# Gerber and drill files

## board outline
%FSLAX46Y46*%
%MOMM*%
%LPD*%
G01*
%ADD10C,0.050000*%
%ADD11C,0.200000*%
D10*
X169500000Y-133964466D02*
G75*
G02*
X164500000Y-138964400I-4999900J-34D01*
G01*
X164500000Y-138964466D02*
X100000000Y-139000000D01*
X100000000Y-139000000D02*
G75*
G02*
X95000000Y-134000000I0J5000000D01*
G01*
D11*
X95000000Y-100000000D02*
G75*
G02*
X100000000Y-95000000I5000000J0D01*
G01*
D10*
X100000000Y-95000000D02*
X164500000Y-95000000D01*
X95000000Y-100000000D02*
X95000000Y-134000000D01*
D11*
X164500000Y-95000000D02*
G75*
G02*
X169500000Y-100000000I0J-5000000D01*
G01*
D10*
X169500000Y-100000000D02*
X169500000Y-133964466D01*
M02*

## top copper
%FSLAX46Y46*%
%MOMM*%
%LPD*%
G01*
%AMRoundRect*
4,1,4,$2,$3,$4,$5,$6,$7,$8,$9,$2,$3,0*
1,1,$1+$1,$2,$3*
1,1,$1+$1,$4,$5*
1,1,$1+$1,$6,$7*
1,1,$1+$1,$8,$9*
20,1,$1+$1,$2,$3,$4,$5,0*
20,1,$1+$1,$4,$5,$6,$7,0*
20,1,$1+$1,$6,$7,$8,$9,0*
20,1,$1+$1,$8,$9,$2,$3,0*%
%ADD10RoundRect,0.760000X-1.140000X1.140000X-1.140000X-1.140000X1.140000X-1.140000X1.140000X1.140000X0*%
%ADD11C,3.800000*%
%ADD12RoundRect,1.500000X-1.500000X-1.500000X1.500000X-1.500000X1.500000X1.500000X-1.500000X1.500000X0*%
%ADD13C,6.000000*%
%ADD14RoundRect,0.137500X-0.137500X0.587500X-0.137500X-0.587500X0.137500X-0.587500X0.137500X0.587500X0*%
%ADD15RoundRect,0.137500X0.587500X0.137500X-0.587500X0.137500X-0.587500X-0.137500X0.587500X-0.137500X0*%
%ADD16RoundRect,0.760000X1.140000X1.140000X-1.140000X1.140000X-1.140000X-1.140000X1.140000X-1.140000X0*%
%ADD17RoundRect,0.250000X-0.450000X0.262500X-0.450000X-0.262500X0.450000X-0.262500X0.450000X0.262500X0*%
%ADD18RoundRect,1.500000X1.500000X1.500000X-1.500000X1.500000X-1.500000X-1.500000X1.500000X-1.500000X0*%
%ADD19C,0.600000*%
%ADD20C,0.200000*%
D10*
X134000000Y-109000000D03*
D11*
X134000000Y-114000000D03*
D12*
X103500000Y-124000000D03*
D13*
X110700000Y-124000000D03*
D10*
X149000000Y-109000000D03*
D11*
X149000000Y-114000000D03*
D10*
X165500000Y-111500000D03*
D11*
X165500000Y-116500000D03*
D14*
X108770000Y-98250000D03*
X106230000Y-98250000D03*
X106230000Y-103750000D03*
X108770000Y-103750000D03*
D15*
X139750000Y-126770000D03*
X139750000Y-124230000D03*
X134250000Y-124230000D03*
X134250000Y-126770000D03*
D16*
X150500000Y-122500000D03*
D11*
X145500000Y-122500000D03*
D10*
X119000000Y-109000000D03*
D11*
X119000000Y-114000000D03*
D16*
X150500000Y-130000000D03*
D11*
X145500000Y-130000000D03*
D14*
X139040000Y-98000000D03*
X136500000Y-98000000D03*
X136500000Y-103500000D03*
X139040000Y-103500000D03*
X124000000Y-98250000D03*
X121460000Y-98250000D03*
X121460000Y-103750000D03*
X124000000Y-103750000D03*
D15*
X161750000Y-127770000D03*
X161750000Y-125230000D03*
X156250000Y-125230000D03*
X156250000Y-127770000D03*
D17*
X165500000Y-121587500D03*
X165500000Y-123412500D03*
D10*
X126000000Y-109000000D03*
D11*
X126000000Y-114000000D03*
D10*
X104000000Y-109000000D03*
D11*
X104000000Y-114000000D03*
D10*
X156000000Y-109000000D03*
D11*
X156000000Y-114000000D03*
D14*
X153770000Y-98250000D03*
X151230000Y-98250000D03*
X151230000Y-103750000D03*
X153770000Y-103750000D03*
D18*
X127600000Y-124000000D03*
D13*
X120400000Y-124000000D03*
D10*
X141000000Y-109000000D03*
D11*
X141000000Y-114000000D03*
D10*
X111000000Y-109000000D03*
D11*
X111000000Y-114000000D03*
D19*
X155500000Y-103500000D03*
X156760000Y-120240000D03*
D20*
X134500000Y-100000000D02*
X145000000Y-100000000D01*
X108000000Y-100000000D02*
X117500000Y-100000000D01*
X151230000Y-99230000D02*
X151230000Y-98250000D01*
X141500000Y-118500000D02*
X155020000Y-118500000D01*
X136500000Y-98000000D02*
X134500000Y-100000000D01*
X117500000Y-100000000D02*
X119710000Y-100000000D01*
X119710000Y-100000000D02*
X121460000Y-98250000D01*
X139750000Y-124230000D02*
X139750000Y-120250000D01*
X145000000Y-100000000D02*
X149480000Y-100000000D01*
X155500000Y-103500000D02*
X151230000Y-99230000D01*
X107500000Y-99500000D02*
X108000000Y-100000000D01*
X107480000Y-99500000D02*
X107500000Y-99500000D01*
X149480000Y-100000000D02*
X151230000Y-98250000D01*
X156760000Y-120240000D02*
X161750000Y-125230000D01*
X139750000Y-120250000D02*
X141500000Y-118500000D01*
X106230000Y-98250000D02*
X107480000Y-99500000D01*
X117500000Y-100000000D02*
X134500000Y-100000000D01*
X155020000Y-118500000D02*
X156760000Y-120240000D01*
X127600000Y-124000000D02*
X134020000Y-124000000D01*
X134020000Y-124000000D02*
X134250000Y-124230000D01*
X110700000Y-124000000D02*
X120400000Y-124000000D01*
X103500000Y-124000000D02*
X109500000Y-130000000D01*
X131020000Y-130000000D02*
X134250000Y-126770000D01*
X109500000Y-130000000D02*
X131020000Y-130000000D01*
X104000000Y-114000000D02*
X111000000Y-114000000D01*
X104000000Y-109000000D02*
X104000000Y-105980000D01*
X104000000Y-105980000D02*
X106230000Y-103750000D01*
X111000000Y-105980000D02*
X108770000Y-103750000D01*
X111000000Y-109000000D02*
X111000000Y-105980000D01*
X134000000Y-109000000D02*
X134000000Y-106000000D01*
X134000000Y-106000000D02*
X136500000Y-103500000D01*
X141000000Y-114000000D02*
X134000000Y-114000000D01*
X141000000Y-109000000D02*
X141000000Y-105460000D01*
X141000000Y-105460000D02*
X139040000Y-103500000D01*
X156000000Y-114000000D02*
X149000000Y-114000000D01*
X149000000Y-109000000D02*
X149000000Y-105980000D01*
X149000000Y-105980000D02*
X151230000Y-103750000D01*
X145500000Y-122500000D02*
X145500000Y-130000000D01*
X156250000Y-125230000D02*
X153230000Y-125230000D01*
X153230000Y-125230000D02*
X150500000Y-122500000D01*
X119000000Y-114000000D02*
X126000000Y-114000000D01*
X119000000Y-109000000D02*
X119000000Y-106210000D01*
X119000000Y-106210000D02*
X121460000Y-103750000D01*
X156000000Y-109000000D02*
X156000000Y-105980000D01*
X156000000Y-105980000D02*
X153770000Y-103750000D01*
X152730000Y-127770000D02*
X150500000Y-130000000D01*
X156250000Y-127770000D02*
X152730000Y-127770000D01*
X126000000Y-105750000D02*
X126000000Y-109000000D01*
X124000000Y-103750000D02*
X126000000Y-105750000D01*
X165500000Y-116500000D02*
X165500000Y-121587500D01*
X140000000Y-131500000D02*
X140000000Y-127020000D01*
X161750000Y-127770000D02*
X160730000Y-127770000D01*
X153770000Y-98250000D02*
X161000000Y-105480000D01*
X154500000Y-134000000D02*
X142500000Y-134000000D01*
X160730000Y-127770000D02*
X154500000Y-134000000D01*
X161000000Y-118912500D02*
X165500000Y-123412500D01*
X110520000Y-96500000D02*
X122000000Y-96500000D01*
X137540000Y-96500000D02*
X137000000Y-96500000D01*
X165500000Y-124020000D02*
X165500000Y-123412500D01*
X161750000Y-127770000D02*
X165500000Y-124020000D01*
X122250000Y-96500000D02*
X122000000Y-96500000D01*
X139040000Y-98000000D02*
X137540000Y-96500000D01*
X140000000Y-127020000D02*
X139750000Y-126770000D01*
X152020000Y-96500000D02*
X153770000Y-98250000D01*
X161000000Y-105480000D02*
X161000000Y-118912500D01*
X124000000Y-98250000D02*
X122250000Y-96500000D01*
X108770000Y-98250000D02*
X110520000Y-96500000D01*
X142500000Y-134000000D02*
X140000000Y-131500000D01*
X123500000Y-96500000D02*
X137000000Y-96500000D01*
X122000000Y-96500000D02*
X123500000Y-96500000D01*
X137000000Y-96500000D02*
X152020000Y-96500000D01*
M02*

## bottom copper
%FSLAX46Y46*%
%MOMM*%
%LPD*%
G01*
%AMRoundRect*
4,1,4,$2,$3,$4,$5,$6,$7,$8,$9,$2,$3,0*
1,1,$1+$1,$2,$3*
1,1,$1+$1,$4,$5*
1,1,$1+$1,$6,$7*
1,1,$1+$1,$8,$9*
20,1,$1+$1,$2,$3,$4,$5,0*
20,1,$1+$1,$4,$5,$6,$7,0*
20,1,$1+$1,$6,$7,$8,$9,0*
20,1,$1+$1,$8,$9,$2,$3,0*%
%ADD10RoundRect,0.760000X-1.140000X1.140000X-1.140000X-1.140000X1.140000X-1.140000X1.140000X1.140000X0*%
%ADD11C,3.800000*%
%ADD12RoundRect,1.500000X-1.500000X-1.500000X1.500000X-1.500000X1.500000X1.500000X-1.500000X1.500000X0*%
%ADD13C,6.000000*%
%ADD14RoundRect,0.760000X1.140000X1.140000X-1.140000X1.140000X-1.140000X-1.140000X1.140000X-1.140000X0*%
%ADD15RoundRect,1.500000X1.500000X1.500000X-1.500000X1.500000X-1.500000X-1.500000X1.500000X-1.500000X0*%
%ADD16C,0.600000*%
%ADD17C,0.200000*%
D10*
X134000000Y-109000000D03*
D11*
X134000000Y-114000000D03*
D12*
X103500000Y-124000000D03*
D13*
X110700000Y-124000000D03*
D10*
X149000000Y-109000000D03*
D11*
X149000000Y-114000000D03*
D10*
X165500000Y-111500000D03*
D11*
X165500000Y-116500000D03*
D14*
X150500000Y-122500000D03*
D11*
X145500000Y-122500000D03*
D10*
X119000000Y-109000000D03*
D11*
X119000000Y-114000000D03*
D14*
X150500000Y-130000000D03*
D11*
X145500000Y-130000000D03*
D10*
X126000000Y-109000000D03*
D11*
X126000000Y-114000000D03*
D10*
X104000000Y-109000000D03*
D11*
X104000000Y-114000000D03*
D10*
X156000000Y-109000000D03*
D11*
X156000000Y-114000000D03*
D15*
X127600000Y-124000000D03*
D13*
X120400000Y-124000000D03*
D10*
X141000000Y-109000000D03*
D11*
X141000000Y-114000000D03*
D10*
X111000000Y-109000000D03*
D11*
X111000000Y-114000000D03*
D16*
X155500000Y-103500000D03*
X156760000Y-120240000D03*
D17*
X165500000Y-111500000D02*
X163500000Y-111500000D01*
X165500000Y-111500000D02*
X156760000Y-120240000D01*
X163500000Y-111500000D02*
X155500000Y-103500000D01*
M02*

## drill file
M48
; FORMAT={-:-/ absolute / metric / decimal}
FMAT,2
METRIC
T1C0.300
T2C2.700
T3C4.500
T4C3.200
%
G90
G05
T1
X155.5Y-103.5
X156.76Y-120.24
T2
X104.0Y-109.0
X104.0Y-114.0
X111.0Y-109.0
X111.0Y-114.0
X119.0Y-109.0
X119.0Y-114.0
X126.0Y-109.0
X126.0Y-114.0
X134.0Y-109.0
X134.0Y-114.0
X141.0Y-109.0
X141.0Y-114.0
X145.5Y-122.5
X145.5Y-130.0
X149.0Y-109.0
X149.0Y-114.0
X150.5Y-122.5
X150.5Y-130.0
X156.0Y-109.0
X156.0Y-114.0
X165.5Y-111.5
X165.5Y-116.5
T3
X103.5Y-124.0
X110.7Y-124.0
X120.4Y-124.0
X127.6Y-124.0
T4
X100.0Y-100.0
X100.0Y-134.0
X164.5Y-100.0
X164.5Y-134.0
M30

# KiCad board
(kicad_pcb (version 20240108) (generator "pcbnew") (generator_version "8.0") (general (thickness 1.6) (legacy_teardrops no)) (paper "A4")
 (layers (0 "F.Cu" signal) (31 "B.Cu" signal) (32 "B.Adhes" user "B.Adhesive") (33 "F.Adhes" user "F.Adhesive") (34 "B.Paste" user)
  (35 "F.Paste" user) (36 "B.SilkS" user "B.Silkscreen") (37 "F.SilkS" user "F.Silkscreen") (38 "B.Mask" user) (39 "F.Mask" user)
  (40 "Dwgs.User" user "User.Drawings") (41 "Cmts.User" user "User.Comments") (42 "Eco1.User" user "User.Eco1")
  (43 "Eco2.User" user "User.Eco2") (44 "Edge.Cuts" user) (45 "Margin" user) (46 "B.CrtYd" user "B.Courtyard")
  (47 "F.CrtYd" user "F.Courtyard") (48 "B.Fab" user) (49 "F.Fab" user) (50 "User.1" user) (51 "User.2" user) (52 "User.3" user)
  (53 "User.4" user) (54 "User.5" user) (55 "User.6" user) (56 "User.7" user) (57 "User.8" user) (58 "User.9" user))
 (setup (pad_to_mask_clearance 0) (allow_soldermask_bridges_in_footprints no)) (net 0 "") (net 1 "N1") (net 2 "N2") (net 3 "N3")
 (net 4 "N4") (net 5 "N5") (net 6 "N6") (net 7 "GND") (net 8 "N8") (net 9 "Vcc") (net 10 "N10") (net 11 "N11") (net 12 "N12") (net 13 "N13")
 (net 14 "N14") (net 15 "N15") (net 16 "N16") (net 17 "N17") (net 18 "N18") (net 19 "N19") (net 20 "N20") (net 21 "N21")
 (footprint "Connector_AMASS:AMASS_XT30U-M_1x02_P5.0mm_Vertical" (layer "F.Cu") (at 134 109 -90)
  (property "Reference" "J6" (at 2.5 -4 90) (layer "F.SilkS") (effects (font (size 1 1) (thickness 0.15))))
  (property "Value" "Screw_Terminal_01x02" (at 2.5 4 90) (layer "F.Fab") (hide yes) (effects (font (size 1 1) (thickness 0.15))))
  (pad "1" thru_hole roundrect (at 0 0 270) (size 3.8 3.8) (drill 2.7) (layers "*.Cu" "*.Mask") (remove_unused_layers no)
   (roundrect_rratio 0.2) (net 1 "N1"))
  (pad "2" thru_hole circle (at 5 0 270) (size 3.8 3.8) (drill 2.7) (layers "*.Cu" "*.Mask") (remove_unused_layers no) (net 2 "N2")))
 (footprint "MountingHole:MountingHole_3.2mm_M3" (layer "F.Cu") (at 100 100)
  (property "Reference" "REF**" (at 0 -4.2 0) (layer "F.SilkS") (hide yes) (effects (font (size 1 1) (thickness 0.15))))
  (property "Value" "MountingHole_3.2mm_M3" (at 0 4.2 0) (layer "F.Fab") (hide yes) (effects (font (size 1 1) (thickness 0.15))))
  (pad "" np_thru_hole circle (at 0 0) (size 3.2 3.2) (drill 3.2) (layers "*.Cu" "*.Mask")))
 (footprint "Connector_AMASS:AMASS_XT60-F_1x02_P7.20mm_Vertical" (layer "F.Cu") (at 103.5 124)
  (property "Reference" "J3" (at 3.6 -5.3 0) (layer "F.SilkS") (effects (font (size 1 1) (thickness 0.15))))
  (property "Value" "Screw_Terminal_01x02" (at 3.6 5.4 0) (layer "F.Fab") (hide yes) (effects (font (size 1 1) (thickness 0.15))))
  (pad "1" thru_hole roundrect (at 0 0) (size 6 6) (drill 4.5) (layers "*.Cu" "*.Mask") (remove_unused_layers no) (roundrect_rratio 0.25)
   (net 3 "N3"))
  (pad "2" thru_hole circle (at 7.2 0) (size 6 6) (drill 4.5) (layers "*.Cu" "*.Mask") (remove_unused_layers no) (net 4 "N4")))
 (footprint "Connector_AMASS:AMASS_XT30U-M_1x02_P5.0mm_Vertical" (layer "F.Cu") (at 149 109 -90)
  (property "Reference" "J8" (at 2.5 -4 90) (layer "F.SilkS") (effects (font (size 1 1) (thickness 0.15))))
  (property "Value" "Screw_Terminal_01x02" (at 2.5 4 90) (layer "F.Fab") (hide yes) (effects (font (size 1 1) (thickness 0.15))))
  (pad "1" thru_hole roundrect (at 0 0 270) (size 3.8 3.8) (drill 2.7) (layers "*.Cu" "*.Mask") (remove_unused_layers no)
   (roundrect_rratio 0.2) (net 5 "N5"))
  (pad "2" thru_hole circle (at 5 0 270) (size 3.8 3.8) (drill 2.7) (layers "*.Cu" "*.Mask") (remove_unused_layers no) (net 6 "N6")))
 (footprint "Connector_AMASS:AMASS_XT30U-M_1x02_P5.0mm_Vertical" (layer "F.Cu") (at 165.5 111.5 -90)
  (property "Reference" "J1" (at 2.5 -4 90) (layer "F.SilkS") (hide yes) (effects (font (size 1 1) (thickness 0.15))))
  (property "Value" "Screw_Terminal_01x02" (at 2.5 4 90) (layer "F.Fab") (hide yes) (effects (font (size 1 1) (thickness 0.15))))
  (pad "1" thru_hole roundrect (at 0 0 270) (size 3.8 3.8) (drill 2.7) (layers "*.Cu" "*.Mask") (remove_unused_layers no)
   (roundrect_rratio 0.2) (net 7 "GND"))
  (pad "2" thru_hole circle (at 5 0 270) (size 3.8 3.8) (drill 2.7) (layers "*.Cu" "*.Mask") (remove_unused_layers no) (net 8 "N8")))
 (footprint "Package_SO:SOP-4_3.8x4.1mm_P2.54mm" (layer "F.Cu") (at 107.5 101 -90)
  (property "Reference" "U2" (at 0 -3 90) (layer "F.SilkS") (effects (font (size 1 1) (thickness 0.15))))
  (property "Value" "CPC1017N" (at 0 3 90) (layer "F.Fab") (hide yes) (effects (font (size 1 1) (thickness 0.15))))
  (pad "1" smd roundrect (at -2.75 -1.27 270) (size 1.45 0.55) (layers "F.Cu" "F.Paste" "F.Mask") (roundrect_rratio 0.25) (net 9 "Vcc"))
  (pad "2" smd roundrect (at -2.75 1.27 270) (size 1.45 0.55) (layers "F.Cu" "F.Paste" "F.Mask") (roundrect_rratio 0.25) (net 7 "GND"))
  (pad "3" smd roundrect (at 2.75 1.27 270) (size 1.45 0.55) (layers "F.Cu" "F.Paste" "F.Mask") (roundrect_rratio 0.25) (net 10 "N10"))
  (pad "4" smd roundrect (at 2.75 -1.27 270) (size 1.45 0.55) (layers "F.Cu" "F.Paste" "F.Mask") (roundrect_rratio 0.25) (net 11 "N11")))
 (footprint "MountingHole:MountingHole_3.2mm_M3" (layer "F.Cu") (at 164.5 134)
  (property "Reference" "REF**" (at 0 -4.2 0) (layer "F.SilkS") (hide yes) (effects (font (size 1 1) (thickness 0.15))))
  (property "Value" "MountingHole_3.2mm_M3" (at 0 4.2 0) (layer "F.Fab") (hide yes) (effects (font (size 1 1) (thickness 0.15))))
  (pad "" np_thru_hole circle (at 0 0) (size 3.2 3.2) (drill 3.2) (layers "*.Cu" "*.Mask")))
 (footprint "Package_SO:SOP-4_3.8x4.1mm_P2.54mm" (layer "F.Cu") (at 137 125.5 180)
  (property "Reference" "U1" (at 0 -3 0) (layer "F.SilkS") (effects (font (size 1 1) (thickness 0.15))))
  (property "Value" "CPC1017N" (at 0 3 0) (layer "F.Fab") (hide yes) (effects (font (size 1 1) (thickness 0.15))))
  (pad "1" smd roundrect (at -2.75 -1.27 180) (size 1.45 0.55) (layers "F.Cu" "F.Paste" "F.Mask") (roundrect_rratio 0.25) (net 9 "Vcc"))
  (pad "2" smd roundrect (at -2.75 1.27 180) (size 1.45 0.55) (layers "F.Cu" "F.Paste" "F.Mask") (roundrect_rratio 0.25) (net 7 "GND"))
  (pad "3" smd roundrect (at 2.75 1.27 180) (size 1.45 0.55) (layers "F.Cu" "F.Paste" "F.Mask") (roundrect_rratio 0.25) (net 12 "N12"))
  (pad "4" smd roundrect (at 2.75 -1.27 180) (size 1.45 0.55) (layers "F.Cu" "F.Paste" "F.Mask") (roundrect_rratio 0.25) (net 3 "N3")))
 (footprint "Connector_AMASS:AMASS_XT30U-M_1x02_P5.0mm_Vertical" (layer "F.Cu") (at 150.5 122.5 180)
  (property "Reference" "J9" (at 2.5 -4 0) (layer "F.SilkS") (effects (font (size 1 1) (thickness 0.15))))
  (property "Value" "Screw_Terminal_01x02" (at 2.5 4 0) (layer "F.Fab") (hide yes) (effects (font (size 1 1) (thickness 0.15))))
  (pad "1" thru_hole roundrect (at 0 0 180) (size 3.8 3.8) (drill 2.7) (layers "*.Cu" "*.Mask") (remove_unused_layers no)
   (roundrect_rratio 0.2) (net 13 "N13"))
  (pad "2" thru_hole circle (at 5 0 180) (size 3.8 3.8) (drill 2.7) (layers "*.Cu" "*.Mask") (remove_unused_layers no) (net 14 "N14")))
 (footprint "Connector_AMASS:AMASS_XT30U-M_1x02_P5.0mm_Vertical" (layer "F.Cu") (at 119 109 -90)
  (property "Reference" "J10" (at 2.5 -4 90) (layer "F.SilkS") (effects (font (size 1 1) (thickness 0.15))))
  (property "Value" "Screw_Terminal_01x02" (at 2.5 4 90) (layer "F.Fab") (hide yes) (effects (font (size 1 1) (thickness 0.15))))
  (pad "1" thru_hole roundrect (at 0 0 270) (size 3.8 3.8) (drill 2.7) (layers "*.Cu" "*.Mask") (remove_unused_layers no)
   (roundrect_rratio 0.2) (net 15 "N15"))
  (pad "2" thru_hole circle (at 5 0 270) (size 3.8 3.8) (drill 2.7) (layers "*.Cu" "*.Mask") (remove_unused_layers no) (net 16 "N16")))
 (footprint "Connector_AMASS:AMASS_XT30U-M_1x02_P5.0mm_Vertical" (layer "F.Cu") (at 150.5 130 180)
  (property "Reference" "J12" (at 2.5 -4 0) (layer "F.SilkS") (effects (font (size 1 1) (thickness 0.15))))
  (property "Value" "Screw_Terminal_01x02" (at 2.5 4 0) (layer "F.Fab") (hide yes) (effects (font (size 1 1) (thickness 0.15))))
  (pad "1" thru_hole roundrect (at 0 0 180) (size 3.8 3.8) (drill 2.7) (layers "*.Cu" "*.Mask") (remove_unused_layers no)
   (roundrect_rratio 0.2) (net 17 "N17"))
  (pad "2" thru_hole circle (at 5 0 180) (size 3.8 3.8) (drill 2.7) (layers "*.Cu" "*.Mask") (remove_unused_layers no) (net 14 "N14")))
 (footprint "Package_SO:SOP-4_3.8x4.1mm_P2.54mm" (layer "F.Cu") (at 137.77 100.75 -90)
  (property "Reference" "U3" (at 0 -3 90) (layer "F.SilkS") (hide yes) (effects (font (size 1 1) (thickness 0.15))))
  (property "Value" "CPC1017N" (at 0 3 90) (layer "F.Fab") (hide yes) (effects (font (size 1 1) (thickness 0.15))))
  (pad "1" smd roundrect (at -2.75 -1.27 270) (size 1.45 0.55) (layers "F.Cu" "F.Paste" "F.Mask") (roundrect_rratio 0.25) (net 9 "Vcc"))
  (pad "2" smd roundrect (at -2.75 1.27 270) (size 1.45 0.55) (layers "F.Cu" "F.Paste" "F.Mask") (roundrect_rratio 0.25) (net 7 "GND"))
  (pad "3" smd roundrect (at 2.75 1.27 270) (size 1.45 0.55) (layers "F.Cu" "F.Paste" "F.Mask") (roundrect_rratio 0.25) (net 1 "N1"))
  (pad "4" smd roundrect (at 2.75 -1.27 270) (size 1.45 0.55) (layers "F.Cu" "F.Paste" "F.Mask") (roundrect_rratio 0.25) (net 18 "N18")))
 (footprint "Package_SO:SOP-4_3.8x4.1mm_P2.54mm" (layer "F.Cu") (at 122.73 101 -90)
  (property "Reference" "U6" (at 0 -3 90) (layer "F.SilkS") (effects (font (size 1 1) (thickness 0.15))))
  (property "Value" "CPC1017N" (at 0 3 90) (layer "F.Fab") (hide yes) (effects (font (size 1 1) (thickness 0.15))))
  (pad "1" smd roundrect (at -2.75 -1.27 270) (size 1.45 0.55) (layers "F.Cu" "F.Paste" "F.Mask") (roundrect_rratio 0.25) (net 9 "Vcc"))
  (pad "2" smd roundrect (at -2.75 1.27 270) (size 1.45 0.55) (layers "F.Cu" "F.Paste" "F.Mask") (roundrect_rratio 0.25) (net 7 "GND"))
  (pad "3" smd roundrect (at 2.75 1.27 270) (size 1.45 0.55) (layers "F.Cu" "F.Paste" "F.Mask") (roundrect_rratio 0.25) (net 15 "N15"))
  (pad "4" smd roundrect (at 2.75 -1.27 270) (size 1.45 0.55) (layers "F.Cu" "F.Paste" "F.Mask") (roundrect_rratio 0.25) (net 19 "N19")))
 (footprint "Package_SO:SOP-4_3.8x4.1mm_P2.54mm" (layer "F.Cu") (at 159 126.5 180)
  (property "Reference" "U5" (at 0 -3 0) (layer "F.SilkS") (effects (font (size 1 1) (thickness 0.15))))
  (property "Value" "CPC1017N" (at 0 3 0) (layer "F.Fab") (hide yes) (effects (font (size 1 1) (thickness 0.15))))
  (pad "1" smd roundrect (at -2.75 -1.27 180) (size 1.45 0.55) (layers "F.Cu" "F.Paste" "F.Mask") (roundrect_rratio 0.25) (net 9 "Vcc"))
  (pad "2" smd roundrect (at -2.75 1.27 180) (size 1.45 0.55) (layers "F.Cu" "F.Paste" "F.Mask") (roundrect_rratio 0.25) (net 7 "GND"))
  (pad "3" smd roundrect (at 2.75 1.27 180) (size 1.45 0.55) (layers "F.Cu" "F.Paste" "F.Mask") (roundrect_rratio 0.25) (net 13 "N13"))
  (pad "4" smd roundrect (at 2.75 -1.27 180) (size 1.45 0.55) (layers "F.Cu" "F.Paste" "F.Mask") (roundrect_rratio 0.25) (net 17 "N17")))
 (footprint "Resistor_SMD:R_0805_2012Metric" (layer "F.Cu") (at 165.5 122.5 -90)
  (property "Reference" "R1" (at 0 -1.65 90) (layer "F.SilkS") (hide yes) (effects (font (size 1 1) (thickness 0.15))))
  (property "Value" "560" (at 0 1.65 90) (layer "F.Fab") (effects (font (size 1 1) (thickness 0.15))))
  (pad "1" smd roundrect (at -0.9125 0 270) (size 1.025 1.4) (layers "F.Cu" "F.Paste" "F.Mask") (roundrect_rratio 0.243902) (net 8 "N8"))
  (pad "2" smd roundrect (at 0.9125 0 270) (size 1.025 1.4) (layers "F.Cu" "F.Paste" "F.Mask") (roundrect_rratio 0.243902) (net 9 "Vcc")))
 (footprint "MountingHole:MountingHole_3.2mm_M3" (layer "F.Cu") (at 100 134)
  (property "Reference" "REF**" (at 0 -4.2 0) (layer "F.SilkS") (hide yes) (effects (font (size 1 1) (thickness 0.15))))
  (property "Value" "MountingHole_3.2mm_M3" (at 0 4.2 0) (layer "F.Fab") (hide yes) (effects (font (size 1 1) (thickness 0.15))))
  (pad "" np_thru_hole circle (at 0 0) (size 3.2 3.2) (drill 3.2) (layers "*.Cu" "*.Mask")))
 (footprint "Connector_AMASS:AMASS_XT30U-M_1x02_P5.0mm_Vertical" (layer "F.Cu") (at 126 109 -90)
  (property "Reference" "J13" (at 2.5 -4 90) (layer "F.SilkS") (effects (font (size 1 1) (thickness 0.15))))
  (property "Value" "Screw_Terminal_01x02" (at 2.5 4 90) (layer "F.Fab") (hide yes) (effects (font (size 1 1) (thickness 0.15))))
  (pad "1" thru_hole roundrect (at 0 0 270) (size 3.8 3.8) (drill 2.7) (layers "*.Cu" "*.Mask") (remove_unused_layers no)
   (roundrect_rratio 0.2) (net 19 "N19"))
  (pad "2" thru_hole circle (at 5 0 270) (size 3.8 3.8) (drill 2.7) (layers "*.Cu" "*.Mask") (remove_unused_layers no) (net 16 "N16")))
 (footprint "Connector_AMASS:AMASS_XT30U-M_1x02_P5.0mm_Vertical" (layer "F.Cu") (at 104 109 -90)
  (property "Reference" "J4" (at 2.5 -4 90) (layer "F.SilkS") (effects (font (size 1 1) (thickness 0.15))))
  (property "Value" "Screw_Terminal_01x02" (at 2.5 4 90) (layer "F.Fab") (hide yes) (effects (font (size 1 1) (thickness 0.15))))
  (pad "1" thru_hole roundrect (at 0 0 270) (size 3.8 3.8) (drill 2.7) (layers "*.Cu" "*.Mask") (remove_unused_layers no)
   (roundrect_rratio 0.2) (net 10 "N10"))
  (pad "2" thru_hole circle (at 5 0 270) (size 3.8 3.8) (drill 2.7) (layers "*.Cu" "*.Mask") (remove_unused_layers no) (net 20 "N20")))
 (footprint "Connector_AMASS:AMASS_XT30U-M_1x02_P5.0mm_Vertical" (layer "F.Cu") (at 156 109 -90)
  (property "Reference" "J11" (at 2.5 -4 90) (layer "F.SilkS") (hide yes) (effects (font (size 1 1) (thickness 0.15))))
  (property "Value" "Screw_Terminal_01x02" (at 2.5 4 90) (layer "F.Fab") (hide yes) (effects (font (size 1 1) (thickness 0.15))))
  (pad "1" thru_hole roundrect (at 0 0 270) (size 3.8 3.8) (drill 2.7) (layers "*.Cu" "*.Mask") (remove_unused_layers no)
   (roundrect_rratio 0.2) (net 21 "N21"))
  (pad "2" thru_hole circle (at 5 0 270) (size 3.8 3.8) (drill 2.7) (layers "*.Cu" "*.Mask") (remove_unused_layers no) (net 6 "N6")))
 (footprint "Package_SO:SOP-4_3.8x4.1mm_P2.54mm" (layer "F.Cu") (at 152.5 101 -90)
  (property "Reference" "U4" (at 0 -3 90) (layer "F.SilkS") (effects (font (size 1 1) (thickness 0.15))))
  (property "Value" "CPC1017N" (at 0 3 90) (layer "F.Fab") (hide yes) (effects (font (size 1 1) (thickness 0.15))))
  (pad "1" smd roundrect (at -2.75 -1.27 270) (size 1.45 0.55) (layers "F.Cu" "F.Paste" "F.Mask") (roundrect_rratio 0.25) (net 9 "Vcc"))
  (pad "2" smd roundrect (at -2.75 1.27 270) (size 1.45 0.55) (layers "F.Cu" "F.Paste" "F.Mask") (roundrect_rratio 0.25) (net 7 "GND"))
  (pad "3" smd roundrect (at 2.75 1.27 270) (size 1.45 0.55) (layers "F.Cu" "F.Paste" "F.Mask") (roundrect_rratio 0.25) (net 5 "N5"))
  (pad "4" smd roundrect (at 2.75 -1.27 270) (size 1.45 0.55) (layers "F.Cu" "F.Paste" "F.Mask") (roundrect_rratio 0.25) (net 21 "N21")))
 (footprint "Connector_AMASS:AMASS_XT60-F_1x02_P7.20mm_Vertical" (layer "F.Cu") (at 127.6 124 180)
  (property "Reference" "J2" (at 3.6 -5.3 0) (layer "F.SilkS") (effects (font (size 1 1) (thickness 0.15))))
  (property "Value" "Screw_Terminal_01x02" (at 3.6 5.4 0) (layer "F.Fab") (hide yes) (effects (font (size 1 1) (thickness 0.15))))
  (pad "1" thru_hole roundrect (at 0 0 180) (size 6 6) (drill 4.5) (layers "*.Cu" "*.Mask") (remove_unused_layers no)
   (roundrect_rratio 0.25) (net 12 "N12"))
  (pad "2" thru_hole circle (at 7.2 0 180) (size 6 6) (drill 4.5) (layers "*.Cu" "*.Mask") (remove_unused_layers no) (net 4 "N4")))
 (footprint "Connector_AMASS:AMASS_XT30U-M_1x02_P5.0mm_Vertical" (layer "F.Cu") (at 141 109 -90)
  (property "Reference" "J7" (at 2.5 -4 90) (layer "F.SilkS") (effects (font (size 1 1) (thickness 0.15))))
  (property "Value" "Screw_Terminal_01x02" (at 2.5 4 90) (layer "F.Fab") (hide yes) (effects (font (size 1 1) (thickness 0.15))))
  (pad "1" thru_hole roundrect (at 0 0 270) (size 3.8 3.8) (drill 2.7) (layers "*.Cu" "*.Mask") (remove_unused_layers no)
   (roundrect_rratio 0.2) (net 18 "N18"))
  (pad "2" thru_hole circle (at 5 0 270) (size 3.8 3.8) (drill 2.7) (layers "*.Cu" "*.Mask") (remove_unused_layers no) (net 2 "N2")))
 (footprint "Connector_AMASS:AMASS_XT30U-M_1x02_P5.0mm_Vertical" (layer "F.Cu") (at 111 109 -90)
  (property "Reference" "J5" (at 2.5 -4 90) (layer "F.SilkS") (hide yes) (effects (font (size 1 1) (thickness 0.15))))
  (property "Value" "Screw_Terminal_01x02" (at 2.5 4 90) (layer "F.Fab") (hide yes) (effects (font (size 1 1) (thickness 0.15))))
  (pad "1" thru_hole roundrect (at 0 0 270) (size 3.8 3.8) (drill 2.7) (layers "*.Cu" "*.Mask") (remove_unused_layers no)
   (roundrect_rratio 0.2) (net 11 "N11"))
  (pad "2" thru_hole circle (at 5 0 270) (size 3.8 3.8) (drill 2.7) (layers "*.Cu" "*.Mask") (remove_unused_layers no) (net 20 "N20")))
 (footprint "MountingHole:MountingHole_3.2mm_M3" (layer "F.Cu") (at 164.5 100)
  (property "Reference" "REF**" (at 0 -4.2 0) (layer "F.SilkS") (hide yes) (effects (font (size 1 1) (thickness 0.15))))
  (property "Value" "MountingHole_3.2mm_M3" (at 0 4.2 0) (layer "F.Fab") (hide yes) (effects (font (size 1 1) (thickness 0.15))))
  (pad "" np_thru_hole circle (at 0 0) (size 3.2 3.2) (drill 3.2) (layers "*.Cu" "*.Mask")))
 (gr_arc (start 169.5 133.964466) (mid 168.035546 137.500022) (end 164.5 138.964466) (stroke (width 0.05) (type default))
  (layer "Edge.Cuts"))
 (gr_line (start 164.5 138.964466) (end 100 139) (stroke (width 0.05) (type default)) (layer "Edge.Cuts"))
 (gr_arc (start 100 139) (mid 96.464466 137.535534) (end 95 134) (stroke (width 0.05) (type default)) (layer "Edge.Cuts"))
 (gr_arc (start 95 100) (mid 96.464466 96.464466) (end 100 95) (stroke (width 0.2) (type default)) (layer "Edge.Cuts"))
 (gr_line (start 100 95) (end 164.5 95) (stroke (width 0.05) (type default)) (layer "Edge.Cuts"))
 (gr_line (start 95 100) (end 95 134) (stroke (width 0.05) (type default)) (layer "Edge.Cuts"))
 (gr_arc (start 164.5 95) (mid 168.035534 96.464466) (end 169.5 100) (stroke (width 0.2) (type default)) (layer "Edge.Cuts"))
 (gr_line (start 169.5 100) (end 169.5 133.964466) (stroke (width 0.05) (type default)) (layer "Edge.Cuts"))
 (segment (start 134.5 100) (end 145 100) (width 0.2) (layer "F.Cu") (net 7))
 (segment (start 108 100) (end 117.5 100) (width 0.2) (layer "F.Cu") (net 7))
 (segment (start 151.23 99.23) (end 151.23 98.25) (width 0.2) (layer "F.Cu") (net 7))
 (segment (start 141.5 118.5) (end 155.02 118.5) (width 0.2) (layer "F.Cu") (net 7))
 (segment (start 136.5 98) (end 134.5 100) (width 0.2) (layer "F.Cu") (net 7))
 (segment (start 117.5 100) (end 119.71 100) (width 0.2) (layer "F.Cu") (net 7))
 (segment (start 119.71 100) (end 121.46 98.25) (width 0.2) (layer "F.Cu") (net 7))
 (segment (start 139.75 124.23) (end 139.75 120.25) (width 0.2) (layer "F.Cu") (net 7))
 (segment (start 145 100) (end 149.48 100) (width 0.2) (layer "F.Cu") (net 7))
 (segment (start 155.5 103.5) (end 151.23 99.23) (width 0.2) (layer "F.Cu") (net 7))
 (segment (start 107.5 99.5) (end 108 100) (width 0.2) (layer "F.Cu") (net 7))
 (segment (start 107.48 99.5) (end 107.5 99.5) (width 0.2) (layer "F.Cu") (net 7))
 (segment (start 149.48 100) (end 151.23 98.25) (width 0.2) (layer "F.Cu") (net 7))
 (segment (start 156.76 120.24) (end 161.75 125.23) (width 0.2) (layer "F.Cu") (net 7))
 (segment (start 139.75 120.25) (end 141.5 118.5) (width 0.2) (layer "F.Cu") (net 7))
 (segment (start 106.23 98.25) (end 107.48 99.5) (width 0.2) (layer "F.Cu") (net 7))
 (segment (start 117.5 100) (end 134.5 100) (width 0.2) (layer "F.Cu") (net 7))
 (segment (start 155.02 118.5) (end 156.76 120.24) (width 0.2) (layer "F.Cu") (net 7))
 (via (at 155.5 103.5) (size 0.6) (drill 0.3) (layers "F.Cu" "B.Cu") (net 7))
 (via (at 156.76 120.24) (size 0.6) (drill 0.3) (layers "F.Cu" "B.Cu") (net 7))
 (segment (start 165.5 111.5) (end 163.5 111.5) (width 0.2) (layer "B.Cu") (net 7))
 (segment (start 165.5 111.5) (end 156.76 120.24) (width 0.2) (layer "B.Cu") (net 7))
 (segment (start 163.5 111.5) (end 155.5 103.5) (width 0.2) (layer "B.Cu") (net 7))
 (segment (start 127.6 124) (end 134.02 124) (width 0.2) (layer "F.Cu") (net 12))
 (segment (start 134.02 124) (end 134.25 124.23) (width 0.2) (layer "F.Cu") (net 12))
 (segment (start 110.7 124) (end 120.4 124) (width 0.2) (layer "F.Cu") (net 4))
 (segment (start 103.5 124) (end 109.5 130) (width 0.2) (layer "F.Cu") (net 3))
 (segment (start 131.02 130) (end 134.25 126.77) (width 0.2) (layer "F.Cu") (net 3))
 (segment (start 109.5 130) (end 131.02 130) (width 0.2) (layer "F.Cu") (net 3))
 (segment (start 104 114) (end 111 114) (width 0.2) (layer "F.Cu") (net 20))
 (segment (start 104 109) (end 104 105.98) (width 0.2) (layer "F.Cu") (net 10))
 (segment (start 104 105.98) (end 106.23 103.75) (width 0.2) (layer "F.Cu") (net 10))
 (segment (start 111 105.98) (end 108.77 103.75) (width 0.2) (layer "F.Cu") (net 11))
 (segment (start 111 109) (end 111 105.98) (width 0.2) (layer "F.Cu") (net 11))
 (segment (start 134 109) (end 134 106) (width 0.2) (layer "F.Cu") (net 1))
 (segment (start 134 106) (end 136.5 103.5) (width 0.2) (layer "F.Cu") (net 1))
 (segment (start 141 114) (end 134 114) (width 0.2) (layer "F.Cu") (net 2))
 (segment (start 141 109) (end 141 105.46) (width 0.2) (layer "F.Cu") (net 18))
 (segment (start 141 105.46) (end 139.04 103.5) (width 0.2) (layer "F.Cu") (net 18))
 (segment (start 156 114) (end 149 114) (width 0.2) (layer "F.Cu") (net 6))
 (segment (start 149 109) (end 149 105.98) (width 0.2) (layer "F.Cu") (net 5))
 (segment (start 149 105.98) (end 151.23 103.75) (width 0.2) (layer "F.Cu") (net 5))
 (segment (start 145.5 122.5) (end 145.5 130) (width 0.2) (layer "F.Cu") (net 14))
 (segment (start 156.25 125.23) (end 153.23 125.23) (width 0.2) (layer "F.Cu") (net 13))
 (segment (start 153.23 125.23) (end 150.5 122.5) (width 0.2) (layer "F.Cu") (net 13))
 (segment (start 119 114) (end 126 114) (width 0.2) (layer "F.Cu") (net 16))
 (segment (start 119 109) (end 119 106.21) (width 0.2) (layer "F.Cu") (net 15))
 (segment (start 119 106.21) (end 121.46 103.75) (width 0.2) (layer "F.Cu") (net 15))
 (segment (start 156 109) (end 156 105.98) (width 0.2) (layer "F.Cu") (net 21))
 (segment (start 156 105.98) (end 153.77 103.75) (width 0.2) (layer "F.Cu") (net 21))
 (segment (start 152.73 127.77) (end 150.5 130) (width 0.2) (layer "F.Cu") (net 17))
 (segment (start 156.25 127.77) (end 152.73 127.77) (width 0.2) (layer "F.Cu") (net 17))
 (segment (start 126 105.75) (end 126 109) (width 0.2) (layer "F.Cu") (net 19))
 (segment (start 124 103.75) (end 126 105.75) (width 0.2) (layer "F.Cu") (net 19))
 (segment (start 165.5 116.5) (end 165.5 121.5875) (width 0.2) (layer "F.Cu") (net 8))
 (segment (start 140 131.5) (end 140 127.02) (width 0.2) (layer "F.Cu") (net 9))
 (segment (start 161.75 127.77) (end 160.73 127.77) (width 0.2) (layer "F.Cu") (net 9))
 (segment (start 153.77 98.25) (end 161 105.48) (width 0.2) (layer "F.Cu") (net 9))
 (segment (start 154.5 134) (end 142.5 134) (width 0.2) (layer "F.Cu") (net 9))
 (segment (start 160.73 127.77) (end 154.5 134) (width 0.2) (layer "F.Cu") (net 9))
 (segment (start 161 118.9125) (end 165.5 123.4125) (width 0.2) (layer "F.Cu") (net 9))
 (segment (start 110.52 96.5) (end 122 96.5) (width 0.2) (layer "F.Cu") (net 9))
 (segment (start 137.54 96.5) (end 137 96.5) (width 0.2) (layer "F.Cu") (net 9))
 (segment (start 165.5 124.02) (end 165.5 123.4125) (width 0.2) (layer "F.Cu") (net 9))
 (segment (start 161.75 127.77) (end 165.5 124.02) (width 0.2) (layer "F.Cu") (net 9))
 (segment (start 122.25 96.5) (end 122 96.5) (width 0.2) (layer "F.Cu") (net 9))
 (segment (start 139.04 98) (end 137.54 96.5) (width 0.2) (layer "F.Cu") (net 9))
 (segment (start 140 127.02) (end 139.75 126.77) (width 0.2) (layer "F.Cu") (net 9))
 (segment (start 152.02 96.5) (end 153.77 98.25) (width 0.2) (layer "F.Cu") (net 9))
 (segment (start 161 105.48) (end 161 118.9125) (width 0.2) (layer "F.Cu") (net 9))
 (segment (start 124 98.25) (end 122.25 96.5) (width 0.2) (layer "F.Cu") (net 9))
 (segment (start 108.77 98.25) (end 110.52 96.5) (width 0.2) (layer "F.Cu") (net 9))
 (segment (start 142.5 134) (end 140 131.5) (width 0.2) (layer "F.Cu") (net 9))
 (segment (start 123.5 96.5) (end 137 96.5) (width 0.2) (layer "F.Cu") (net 9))
 (segment (start 122 96.5) (end 123.5 96.5) (width 0.2) (layer "F.Cu") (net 9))
 (segment (start 137 96.5) (end 152.02 96.5) (width 0.2) (layer "F.Cu") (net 9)))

